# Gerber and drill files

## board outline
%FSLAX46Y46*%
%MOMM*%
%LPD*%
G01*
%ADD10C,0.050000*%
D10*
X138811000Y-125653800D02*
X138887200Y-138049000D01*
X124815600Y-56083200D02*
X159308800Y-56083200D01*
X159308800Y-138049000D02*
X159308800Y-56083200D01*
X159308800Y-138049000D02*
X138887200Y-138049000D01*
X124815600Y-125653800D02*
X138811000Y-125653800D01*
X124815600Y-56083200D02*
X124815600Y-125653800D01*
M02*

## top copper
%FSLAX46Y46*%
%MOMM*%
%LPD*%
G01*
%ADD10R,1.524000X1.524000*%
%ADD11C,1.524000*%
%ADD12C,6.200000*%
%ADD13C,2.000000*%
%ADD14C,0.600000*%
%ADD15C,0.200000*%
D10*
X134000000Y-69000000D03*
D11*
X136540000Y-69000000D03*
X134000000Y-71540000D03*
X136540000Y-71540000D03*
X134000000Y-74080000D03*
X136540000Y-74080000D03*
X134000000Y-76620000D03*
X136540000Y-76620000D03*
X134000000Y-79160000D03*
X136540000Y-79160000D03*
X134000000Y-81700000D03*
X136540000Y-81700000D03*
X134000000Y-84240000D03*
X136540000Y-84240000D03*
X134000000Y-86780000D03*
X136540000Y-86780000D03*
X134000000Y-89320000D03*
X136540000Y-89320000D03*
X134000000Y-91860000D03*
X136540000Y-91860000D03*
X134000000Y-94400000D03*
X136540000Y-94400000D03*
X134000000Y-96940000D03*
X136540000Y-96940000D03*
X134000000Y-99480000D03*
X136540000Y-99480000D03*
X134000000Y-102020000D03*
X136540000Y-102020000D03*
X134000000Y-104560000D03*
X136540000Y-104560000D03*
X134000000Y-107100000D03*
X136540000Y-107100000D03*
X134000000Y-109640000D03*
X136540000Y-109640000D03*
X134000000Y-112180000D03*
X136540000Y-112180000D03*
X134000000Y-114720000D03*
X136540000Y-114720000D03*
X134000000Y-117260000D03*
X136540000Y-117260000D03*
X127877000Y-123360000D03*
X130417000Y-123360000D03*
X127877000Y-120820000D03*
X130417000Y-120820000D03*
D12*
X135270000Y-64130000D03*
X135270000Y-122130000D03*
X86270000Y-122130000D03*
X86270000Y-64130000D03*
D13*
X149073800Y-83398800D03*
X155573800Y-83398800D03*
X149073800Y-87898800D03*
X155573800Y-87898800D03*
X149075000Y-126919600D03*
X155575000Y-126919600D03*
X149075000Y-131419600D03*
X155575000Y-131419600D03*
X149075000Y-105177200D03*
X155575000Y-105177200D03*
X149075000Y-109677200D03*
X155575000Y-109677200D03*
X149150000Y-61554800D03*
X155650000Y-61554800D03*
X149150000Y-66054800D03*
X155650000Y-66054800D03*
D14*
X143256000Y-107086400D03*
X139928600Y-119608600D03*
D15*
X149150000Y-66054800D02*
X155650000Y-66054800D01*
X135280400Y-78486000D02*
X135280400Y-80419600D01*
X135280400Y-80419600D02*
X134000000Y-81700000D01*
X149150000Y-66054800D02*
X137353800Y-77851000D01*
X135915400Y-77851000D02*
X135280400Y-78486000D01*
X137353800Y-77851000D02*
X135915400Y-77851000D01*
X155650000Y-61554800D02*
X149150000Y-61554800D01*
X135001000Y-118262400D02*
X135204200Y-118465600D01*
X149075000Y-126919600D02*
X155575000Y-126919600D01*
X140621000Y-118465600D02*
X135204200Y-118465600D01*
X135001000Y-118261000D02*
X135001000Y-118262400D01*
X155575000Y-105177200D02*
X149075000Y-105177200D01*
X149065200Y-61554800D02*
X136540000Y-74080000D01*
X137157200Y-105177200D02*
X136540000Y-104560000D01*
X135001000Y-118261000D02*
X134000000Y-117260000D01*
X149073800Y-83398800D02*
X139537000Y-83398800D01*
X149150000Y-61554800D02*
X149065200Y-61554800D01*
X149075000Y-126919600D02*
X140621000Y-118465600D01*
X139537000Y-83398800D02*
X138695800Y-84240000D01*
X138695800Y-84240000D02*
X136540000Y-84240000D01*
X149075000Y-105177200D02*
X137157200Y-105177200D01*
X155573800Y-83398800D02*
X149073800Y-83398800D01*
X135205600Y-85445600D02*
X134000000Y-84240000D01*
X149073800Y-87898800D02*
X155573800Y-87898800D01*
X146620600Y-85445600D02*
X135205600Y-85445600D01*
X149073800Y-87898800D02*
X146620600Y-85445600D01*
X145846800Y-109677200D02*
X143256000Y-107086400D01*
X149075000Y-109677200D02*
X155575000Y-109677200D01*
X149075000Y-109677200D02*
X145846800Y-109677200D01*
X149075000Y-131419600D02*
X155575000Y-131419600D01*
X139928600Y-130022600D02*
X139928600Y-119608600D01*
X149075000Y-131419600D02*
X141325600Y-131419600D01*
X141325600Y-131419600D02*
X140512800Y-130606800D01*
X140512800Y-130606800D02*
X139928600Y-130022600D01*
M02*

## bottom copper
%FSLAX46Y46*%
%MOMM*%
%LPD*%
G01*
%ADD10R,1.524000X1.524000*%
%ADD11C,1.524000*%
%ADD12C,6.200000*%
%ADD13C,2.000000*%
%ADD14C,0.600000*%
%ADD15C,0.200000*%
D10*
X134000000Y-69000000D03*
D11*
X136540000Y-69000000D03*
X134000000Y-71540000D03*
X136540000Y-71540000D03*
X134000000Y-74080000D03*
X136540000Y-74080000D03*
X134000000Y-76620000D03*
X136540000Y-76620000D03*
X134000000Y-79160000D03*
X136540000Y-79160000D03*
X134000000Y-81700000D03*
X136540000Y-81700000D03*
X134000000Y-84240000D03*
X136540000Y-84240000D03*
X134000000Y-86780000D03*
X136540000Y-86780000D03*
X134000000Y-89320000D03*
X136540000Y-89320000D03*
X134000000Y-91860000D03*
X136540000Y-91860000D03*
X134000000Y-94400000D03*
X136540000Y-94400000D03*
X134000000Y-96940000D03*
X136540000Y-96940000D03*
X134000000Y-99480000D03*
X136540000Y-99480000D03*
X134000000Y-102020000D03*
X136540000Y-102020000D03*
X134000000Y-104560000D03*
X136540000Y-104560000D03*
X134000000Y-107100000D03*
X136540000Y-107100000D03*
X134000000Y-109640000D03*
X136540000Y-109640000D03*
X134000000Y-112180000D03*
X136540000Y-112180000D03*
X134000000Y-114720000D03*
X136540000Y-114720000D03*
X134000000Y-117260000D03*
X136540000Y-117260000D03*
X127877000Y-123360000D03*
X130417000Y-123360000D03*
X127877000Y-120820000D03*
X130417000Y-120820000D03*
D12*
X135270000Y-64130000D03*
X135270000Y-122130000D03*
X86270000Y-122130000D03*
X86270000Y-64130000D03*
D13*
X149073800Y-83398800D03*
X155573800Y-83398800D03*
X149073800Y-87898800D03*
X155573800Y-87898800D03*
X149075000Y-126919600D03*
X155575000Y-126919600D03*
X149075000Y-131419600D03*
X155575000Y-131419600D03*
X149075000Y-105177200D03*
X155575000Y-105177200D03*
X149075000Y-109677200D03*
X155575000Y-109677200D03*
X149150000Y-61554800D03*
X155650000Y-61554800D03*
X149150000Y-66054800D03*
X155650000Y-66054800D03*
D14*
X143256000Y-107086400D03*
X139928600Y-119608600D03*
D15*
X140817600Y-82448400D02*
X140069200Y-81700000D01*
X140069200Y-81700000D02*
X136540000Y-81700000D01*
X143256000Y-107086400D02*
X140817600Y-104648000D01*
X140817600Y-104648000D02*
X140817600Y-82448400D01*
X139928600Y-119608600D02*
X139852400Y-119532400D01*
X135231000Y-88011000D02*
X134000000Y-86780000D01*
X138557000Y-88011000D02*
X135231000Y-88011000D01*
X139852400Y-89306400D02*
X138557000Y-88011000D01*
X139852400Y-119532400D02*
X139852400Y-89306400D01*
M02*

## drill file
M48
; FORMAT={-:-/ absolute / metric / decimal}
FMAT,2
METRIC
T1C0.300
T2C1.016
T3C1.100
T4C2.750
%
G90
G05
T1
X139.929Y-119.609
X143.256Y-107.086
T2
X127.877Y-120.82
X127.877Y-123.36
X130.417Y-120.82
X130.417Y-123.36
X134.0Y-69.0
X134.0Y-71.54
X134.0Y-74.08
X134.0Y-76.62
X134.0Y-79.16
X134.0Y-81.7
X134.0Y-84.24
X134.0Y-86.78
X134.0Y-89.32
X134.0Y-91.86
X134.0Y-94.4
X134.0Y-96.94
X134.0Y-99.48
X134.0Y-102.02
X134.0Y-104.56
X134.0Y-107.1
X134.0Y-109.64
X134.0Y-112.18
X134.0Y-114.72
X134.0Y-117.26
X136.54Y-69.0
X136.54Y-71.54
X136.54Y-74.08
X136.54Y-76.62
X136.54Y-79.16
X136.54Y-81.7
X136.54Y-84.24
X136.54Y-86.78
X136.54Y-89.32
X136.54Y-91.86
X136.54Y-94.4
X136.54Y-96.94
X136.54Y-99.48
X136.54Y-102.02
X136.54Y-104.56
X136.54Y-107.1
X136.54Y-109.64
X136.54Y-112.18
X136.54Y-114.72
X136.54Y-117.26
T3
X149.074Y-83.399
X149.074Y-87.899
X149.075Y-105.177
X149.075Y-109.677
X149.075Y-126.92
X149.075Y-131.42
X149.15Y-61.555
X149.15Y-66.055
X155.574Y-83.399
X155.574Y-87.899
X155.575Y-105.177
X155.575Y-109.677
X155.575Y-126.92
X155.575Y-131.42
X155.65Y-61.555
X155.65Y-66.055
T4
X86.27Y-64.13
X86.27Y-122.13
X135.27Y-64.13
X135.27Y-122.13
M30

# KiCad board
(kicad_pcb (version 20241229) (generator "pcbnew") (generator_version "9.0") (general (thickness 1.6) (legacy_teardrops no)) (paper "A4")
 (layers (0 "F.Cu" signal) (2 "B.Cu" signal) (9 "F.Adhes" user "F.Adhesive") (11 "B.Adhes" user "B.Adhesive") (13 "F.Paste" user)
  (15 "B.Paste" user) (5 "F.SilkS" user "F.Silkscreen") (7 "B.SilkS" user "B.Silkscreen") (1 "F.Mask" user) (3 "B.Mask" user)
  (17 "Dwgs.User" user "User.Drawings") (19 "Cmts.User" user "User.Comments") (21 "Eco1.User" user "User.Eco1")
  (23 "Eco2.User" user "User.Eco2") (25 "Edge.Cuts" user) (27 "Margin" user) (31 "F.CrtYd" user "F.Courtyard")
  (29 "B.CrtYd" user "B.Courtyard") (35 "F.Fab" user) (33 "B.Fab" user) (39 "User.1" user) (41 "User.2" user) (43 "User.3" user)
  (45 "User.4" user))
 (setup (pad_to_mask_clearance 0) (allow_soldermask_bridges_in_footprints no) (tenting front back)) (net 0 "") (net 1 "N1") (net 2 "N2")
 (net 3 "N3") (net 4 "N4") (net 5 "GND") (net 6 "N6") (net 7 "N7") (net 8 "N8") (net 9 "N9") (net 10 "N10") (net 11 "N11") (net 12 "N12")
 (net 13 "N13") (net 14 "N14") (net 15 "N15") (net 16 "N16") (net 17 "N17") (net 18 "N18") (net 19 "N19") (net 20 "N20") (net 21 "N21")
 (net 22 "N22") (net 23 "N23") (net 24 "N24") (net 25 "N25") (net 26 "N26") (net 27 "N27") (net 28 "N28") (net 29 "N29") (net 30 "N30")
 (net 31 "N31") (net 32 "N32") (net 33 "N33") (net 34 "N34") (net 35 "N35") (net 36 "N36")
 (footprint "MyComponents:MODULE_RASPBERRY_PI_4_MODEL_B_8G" (layer "F.Cu") (at 110.77 103.13 -90)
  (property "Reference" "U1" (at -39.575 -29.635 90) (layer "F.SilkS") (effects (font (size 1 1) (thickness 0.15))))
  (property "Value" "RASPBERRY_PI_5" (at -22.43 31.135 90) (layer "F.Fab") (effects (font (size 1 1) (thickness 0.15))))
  (pad "1" thru_hole rect (at -34.13 -23.23 270) (size 1.524 1.524) (drill 1.016) (layers "*.Cu" "*.Mask") (remove_unused_layers no)
   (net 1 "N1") (solder_mask_margin 0.102))
  (pad "2" thru_hole circle (at -34.13 -25.77 270) (size 1.524 1.524) (drill 1.016) (layers "*.Cu" "*.Mask") (remove_unused_layers no)
   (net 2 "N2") (solder_mask_margin 0.102))
  (pad "3" thru_hole circle (at -31.59 -23.23 270) (size 1.524 1.524) (drill 1.016) (layers "*.Cu" "*.Mask") (remove_unused_layers no)
   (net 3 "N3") (solder_mask_margin 0.102))
  (pad "4" thru_hole circle (at -31.59 -25.77 270) (size 1.524 1.524) (drill 1.016) (layers "*.Cu" "*.Mask") (remove_unused_layers no)
   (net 2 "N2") (solder_mask_margin 0.102))
  (pad "5" thru_hole circle (at -29.05 -23.23 270) (size 1.524 1.524) (drill 1.016) (layers "*.Cu" "*.Mask") (remove_unused_layers no)
   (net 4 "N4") (solder_mask_margin 0.102))
  (pad "6" thru_hole circle (at -29.05 -25.77 270) (size 1.524 1.524) (drill 1.016) (layers "*.Cu" "*.Mask") (remove_unused_layers no)
   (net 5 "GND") (solder_mask_margin 0.102))
  (pad "7" thru_hole circle (at -26.51 -23.23 270) (size 1.524 1.524) (drill 1.016) (layers "*.Cu" "*.Mask") (remove_unused_layers no)
   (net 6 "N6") (solder_mask_margin 0.102))
  (pad "8" thru_hole circle (at -26.51 -25.77 270) (size 1.524 1.524) (drill 1.016) (layers "*.Cu" "*.Mask") (remove_unused_layers no)
   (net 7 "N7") (solder_mask_margin 0.102))
  (pad "9" thru_hole circle (at -23.97 -23.23 270) (size 1.524 1.524) (drill 1.016) (layers "*.Cu" "*.Mask") (remove_unused_layers no)
   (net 5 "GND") (solder_mask_margin 0.102))
  (pad "10" thru_hole circle (at -23.97 -25.77 270) (size 1.524 1.524) (drill 1.016) (layers "*.Cu" "*.Mask") (remove_unused_layers no)
   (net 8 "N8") (solder_mask_margin 0.102))
  (pad "11" thru_hole circle (at -21.43 -23.23 270) (size 1.524 1.524) (drill 1.016) (layers "*.Cu" "*.Mask") (remove_unused_layers no)
   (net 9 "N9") (solder_mask_margin 0.102))
  (pad "12" thru_hole circle (at -21.43 -25.77 270) (size 1.524 1.524) (drill 1.016) (layers "*.Cu" "*.Mask") (remove_unused_layers no)
   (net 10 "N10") (solder_mask_margin 0.102))
  (pad "13" thru_hole circle (at -18.89 -23.23 270) (size 1.524 1.524) (drill 1.016) (layers "*.Cu" "*.Mask") (remove_unused_layers no)
   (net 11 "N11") (solder_mask_margin 0.102))
  (pad "14" thru_hole circle (at -18.89 -25.77 270) (size 1.524 1.524) (drill 1.016) (layers "*.Cu" "*.Mask") (remove_unused_layers no)
   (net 5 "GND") (solder_mask_margin 0.102))
  (pad "15" thru_hole circle (at -16.35 -23.23 270) (size 1.524 1.524) (drill 1.016) (layers "*.Cu" "*.Mask") (remove_unused_layers no)
   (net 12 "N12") (solder_mask_margin 0.102))
  (pad "16" thru_hole circle (at -16.35 -25.77 270) (size 1.524 1.524) (drill 1.016) (layers "*.Cu" "*.Mask") (remove_unused_layers no)
   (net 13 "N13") (solder_mask_margin 0.102))
  (pad "17" thru_hole circle (at -13.81 -23.23 270) (size 1.524 1.524) (drill 1.016) (layers "*.Cu" "*.Mask") (remove_unused_layers no)
   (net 1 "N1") (solder_mask_margin 0.102))
  (pad "18" thru_hole circle (at -13.81 -25.77 270) (size 1.524 1.524) (drill 1.016) (layers "*.Cu" "*.Mask") (remove_unused_layers no)
   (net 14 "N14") (solder_mask_margin 0.102))
  (pad "19" thru_hole circle (at -11.27 -23.23 270) (size 1.524 1.524) (drill 1.016) (layers "*.Cu" "*.Mask") (remove_unused_layers no)
   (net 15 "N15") (solder_mask_margin 0.102))
  (pad "20" thru_hole circle (at -11.27 -25.77 270) (size 1.524 1.524) (drill 1.016) (layers "*.Cu" "*.Mask") (remove_unused_layers no)
   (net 5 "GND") (solder_mask_margin 0.102))
  (pad "21" thru_hole circle (at -8.73 -23.23 270) (size 1.524 1.524) (drill 1.016) (layers "*.Cu" "*.Mask") (remove_unused_layers no)
   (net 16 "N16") (solder_mask_margin 0.102))
  (pad "22" thru_hole circle (at -8.73 -25.77 270) (size 1.524 1.524) (drill 1.016) (layers "*.Cu" "*.Mask") (remove_unused_layers no)
   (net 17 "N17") (solder_mask_margin 0.102))
  (pad "23" thru_hole circle (at -6.19 -23.23 270) (size 1.524 1.524) (drill 1.016) (layers "*.Cu" "*.Mask") (remove_unused_layers no)
   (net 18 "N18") (solder_mask_margin 0.102))
  (pad "24" thru_hole circle (at -6.19 -25.77 270) (size 1.524 1.524) (drill 1.016) (layers "*.Cu" "*.Mask") (remove_unused_layers no)
   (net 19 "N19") (solder_mask_margin 0.102))
  (pad "25" thru_hole circle (at -3.65 -23.23 270) (size 1.524 1.524) (drill 1.016) (layers "*.Cu" "*.Mask") (remove_unused_layers no)
   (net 5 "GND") (solder_mask_margin 0.102))
  (pad "26" thru_hole circle (at -3.65 -25.77 270) (size 1.524 1.524) (drill 1.016) (layers "*.Cu" "*.Mask") (remove_unused_layers no)
   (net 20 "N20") (solder_mask_margin 0.102))
  (pad "27" thru_hole circle (at -1.11 -23.23 270) (size 1.524 1.524) (drill 1.016) (layers "*.Cu" "*.Mask") (remove_unused_layers no)
   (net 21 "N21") (solder_mask_margin 0.102))
  (pad "28" thru_hole circle (at -1.11 -25.77 270) (size 1.524 1.524) (drill 1.016) (layers "*.Cu" "*.Mask") (remove_unused_layers no)
   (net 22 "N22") (solder_mask_margin 0.102))
  (pad "29" thru_hole circle (at 1.43 -23.23 270) (size 1.524 1.524) (drill 1.016) (layers "*.Cu" "*.Mask") (remove_unused_layers no)
   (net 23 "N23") (solder_mask_margin 0.102))
  (pad "30" thru_hole circle (at 1.43 -25.77 270) (size 1.524 1.524) (drill 1.016) (layers "*.Cu" "*.Mask") (remove_unused_layers no)
   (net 5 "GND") (solder_mask_margin 0.102))
  (pad "31" thru_hole circle (at 3.97 -23.23 270) (size 1.524 1.524) (drill 1.016) (layers "*.Cu" "*.Mask") (remove_unused_layers no)
   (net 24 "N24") (solder_mask_margin 0.102))
  (pad "32" thru_hole circle (at 3.97 -25.77 270) (size 1.524 1.524) (drill 1.016) (layers "*.Cu" "*.Mask") (remove_unused_layers no)
   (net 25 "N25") (solder_mask_margin 0.102))
  (pad "33" thru_hole circle (at 6.51 -23.23 270) (size 1.524 1.524) (drill 1.016) (layers "*.Cu" "*.Mask") (remove_unused_layers no)
   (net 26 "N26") (solder_mask_margin 0.102))
  (pad "34" thru_hole circle (at 6.51 -25.77 270) (size 1.524 1.524) (drill 1.016) (layers "*.Cu" "*.Mask") (remove_unused_layers no)
   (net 5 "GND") (solder_mask_margin 0.102))
  (pad "35" thru_hole circle (at 9.05 -23.23 270) (size 1.524 1.524) (drill 1.016) (layers "*.Cu" "*.Mask") (remove_unused_layers no)
   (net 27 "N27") (solder_mask_margin 0.102))
  (pad "36" thru_hole circle (at 9.05 -25.77 270) (size 1.524 1.524) (drill 1.016) (layers "*.Cu" "*.Mask") (remove_unused_layers no)
   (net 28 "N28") (solder_mask_margin 0.102))
  (pad "37" thru_hole circle (at 11.59 -23.23 270) (size 1.524 1.524) (drill 1.016) (layers "*.Cu" "*.Mask") (remove_unused_layers no)
   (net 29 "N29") (solder_mask_margin 0.102))
  (pad "38" thru_hole circle (at 11.59 -25.77 270) (size 1.524 1.524) (drill 1.016) (layers "*.Cu" "*.Mask") (remove_unused_layers no)
   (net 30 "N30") (solder_mask_margin 0.102))
  (pad "39" thru_hole circle (at 14.13 -23.23 270) (size 1.524 1.524) (drill 1.016) (layers "*.Cu" "*.Mask") (remove_unused_layers no)
   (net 5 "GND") (solder_mask_margin 0.102))
  (pad "40" thru_hole circle (at 14.13 -25.77 270) (size 1.524 1.524) (drill 1.016) (layers "*.Cu" "*.Mask") (remove_unused_layers no)
   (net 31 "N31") (solder_mask_margin 0.102))
  (pad "41" thru_hole circle (at 20.23 -17.107 270) (size 1.524 1.524) (drill 1.016) (layers "*.Cu" "*.Mask") (remove_unused_layers no)
   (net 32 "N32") (solder_mask_margin 0.102))
  (pad "42" thru_hole circle (at 20.23 -19.647 270) (size 1.524 1.524) (drill 1.016) (layers "*.Cu" "*.Mask") (remove_unused_layers no)
   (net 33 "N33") (solder_mask_margin 0.102))
  (pad "43" thru_hole circle (at 17.69 -17.107 270) (size 1.524 1.524) (drill 1.016) (layers "*.Cu" "*.Mask") (remove_unused_layers no)
   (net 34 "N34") (solder_mask_margin 0.102))
  (pad "44" thru_hole circle (at 17.69 -19.647 270) (size 1.524 1.524) (drill 1.016) (layers "*.Cu" "*.Mask") (remove_unused_layers no)
   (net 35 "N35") (solder_mask_margin 0.102))
  (pad "S1" thru_hole circle (at -39 -24.5 270) (size 6.2 6.2) (drill 2.75) (layers "*.Cu" "*.Mask") (remove_unused_layers no)
   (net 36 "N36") (solder_mask_margin 0.102))
  (pad "S2" thru_hole circle (at 19 -24.5 270) (size 6.2 6.2) (drill 2.75) (layers "*.Cu" "*.Mask") (remove_unused_layers no) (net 36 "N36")
   (solder_mask_margin 0.102))
  (pad "S3" thru_hole circle (at 19 24.5 270) (size 6.2 6.2) (drill 2.75) (layers "*.Cu" "*.Mask") (remove_unused_layers no) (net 36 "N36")
   (solder_mask_margin 0.102))
  (pad "S4" thru_hole circle (at -39 24.5 270) (size 6.2 6.2) (drill 2.75) (layers "*.Cu" "*.Mask") (remove_unused_layers no) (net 36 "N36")
   (solder_mask_margin 0.102)))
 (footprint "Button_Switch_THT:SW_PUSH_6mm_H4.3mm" (layer "F.Cu") (at 149.0738 83.3988)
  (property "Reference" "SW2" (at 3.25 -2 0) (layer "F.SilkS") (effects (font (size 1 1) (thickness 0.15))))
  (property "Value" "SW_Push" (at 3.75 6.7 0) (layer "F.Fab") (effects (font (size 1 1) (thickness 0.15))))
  (pad "1" thru_hole circle (at 0 0 90) (size 2 2) (drill 1.1) (layers "*.Cu" "*.Mask") (remove_unused_layers no) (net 5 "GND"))
  (pad "1" thru_hole circle (at 6.5 0 90) (size 2 2) (drill 1.1) (layers "*.Cu" "*.Mask") (remove_unused_layers no) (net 5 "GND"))
  (pad "2" thru_hole circle (at 0 4.5 90) (size 2 2) (drill 1.1) (layers "*.Cu" "*.Mask") (remove_unused_layers no) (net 11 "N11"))
  (pad "2" thru_hole circle (at 6.5 4.5 90) (size 2 2) (drill 1.1) (layers "*.Cu" "*.Mask") (remove_unused_layers no) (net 11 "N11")))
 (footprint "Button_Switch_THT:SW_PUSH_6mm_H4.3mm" (layer "F.Cu") (at 149.075 126.9196)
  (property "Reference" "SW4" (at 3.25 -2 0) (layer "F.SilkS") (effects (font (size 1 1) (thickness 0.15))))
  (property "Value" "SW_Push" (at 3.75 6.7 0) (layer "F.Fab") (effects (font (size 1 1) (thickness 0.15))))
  (pad "1" thru_hole circle (at 0 0 90) (size 2 2) (drill 1.1) (layers "*.Cu" "*.Mask") (remove_unused_layers no) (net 5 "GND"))
  (pad "1" thru_hole circle (at 6.5 0 90) (size 2 2) (drill 1.1) (layers "*.Cu" "*.Mask") (remove_unused_layers no) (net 5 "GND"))
  (pad "2" thru_hole circle (at 0 4.5 90) (size 2 2) (drill 1.1) (layers "*.Cu" "*.Mask") (remove_unused_layers no) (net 12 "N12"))
  (pad "2" thru_hole circle (at 6.5 4.5 90) (size 2 2) (drill 1.1) (layers "*.Cu" "*.Mask") (remove_unused_layers no) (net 12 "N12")))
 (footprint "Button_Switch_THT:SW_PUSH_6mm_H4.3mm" (layer "F.Cu") (at 149.075 105.1772)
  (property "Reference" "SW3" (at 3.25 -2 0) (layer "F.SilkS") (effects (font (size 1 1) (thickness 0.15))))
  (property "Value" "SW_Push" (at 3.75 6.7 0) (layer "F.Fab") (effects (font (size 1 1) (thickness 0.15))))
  (pad "1" thru_hole circle (at 0 0 90) (size 2 2) (drill 1.1) (layers "*.Cu" "*.Mask") (remove_unused_layers no) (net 5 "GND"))
  (pad "1" thru_hole circle (at 6.5 0 90) (size 2 2) (drill 1.1) (layers "*.Cu" "*.Mask") (remove_unused_layers no) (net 5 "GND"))
  (pad "2" thru_hole circle (at 0 4.5 90) (size 2 2) (drill 1.1) (layers "*.Cu" "*.Mask") (remove_unused_layers no) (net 10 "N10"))
  (pad "2" thru_hole circle (at 6.5 4.5 90) (size 2 2) (drill 1.1) (layers "*.Cu" "*.Mask") (remove_unused_layers no) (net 10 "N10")))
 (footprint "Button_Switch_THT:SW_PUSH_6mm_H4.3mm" (layer "F.Cu") (at 149.15 61.5548)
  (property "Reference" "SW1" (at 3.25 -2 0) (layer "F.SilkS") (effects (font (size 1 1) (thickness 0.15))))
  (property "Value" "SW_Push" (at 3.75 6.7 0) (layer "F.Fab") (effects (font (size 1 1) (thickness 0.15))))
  (pad "1" thru_hole circle (at 0 0 90) (size 2 2) (drill 1.1) (layers "*.Cu" "*.Mask") (remove_unused_layers no) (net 5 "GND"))
  (pad "1" thru_hole circle (at 6.5 0 90) (size 2 2) (drill 1.1) (layers "*.Cu" "*.Mask") (remove_unused_layers no) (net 5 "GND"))
  (pad "2" thru_hole circle (at 0 4.5 90) (size 2 2) (drill 1.1) (layers "*.Cu" "*.Mask") (remove_unused_layers no) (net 9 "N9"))
  (pad "2" thru_hole circle (at 6.5 4.5 90) (size 2 2) (drill 1.1) (layers "*.Cu" "*.Mask") (remove_unused_layers no) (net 9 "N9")))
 (gr_line (start 138.811 125.6538) (end 138.8872 138.049) (stroke (width 0.05) (type default)) (layer "Edge.Cuts"))
 (gr_line (start 124.8156 56.0832) (end 159.3088 56.0832) (stroke (width 0.05) (type default)) (layer "Edge.Cuts"))
 (gr_line (start 159.3088 138.049) (end 159.3088 56.0832) (stroke (width 0.05) (type default)) (layer "Edge.Cuts"))
 (gr_line (start 159.3088 138.049) (end 138.8872 138.049) (stroke (width 0.05) (type default)) (layer "Edge.Cuts"))
 (gr_line (start 124.8156 125.6538) (end 138.811 125.6538) (stroke (width 0.05) (type default)) (layer "Edge.Cuts"))
 (gr_line (start 124.8156 56.0832) (end 124.8156 125.6538) (stroke (width 0.05) (type default)) (layer "Edge.Cuts"))
 (segment (start 149.15 66.0548) (end 155.65 66.0548) (width 0.2) (layer "F.Cu") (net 9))
 (segment (start 135.2804 78.486) (end 135.2804 80.4196) (width 0.2) (layer "F.Cu") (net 9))
 (segment (start 135.2804 80.4196) (end 134 81.7) (width 0.2) (layer "F.Cu") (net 9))
 (segment (start 149.15 66.0548) (end 137.3538 77.851) (width 0.2) (layer "F.Cu") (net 9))
 (segment (start 135.9154 77.851) (end 135.2804 78.486) (width 0.2) (layer "F.Cu") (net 9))
 (segment (start 137.3538 77.851) (end 135.9154 77.851) (width 0.2) (layer "F.Cu") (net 9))
 (segment (start 155.65 61.5548) (end 149.15 61.5548) (width 0.2) (layer "F.Cu") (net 5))
 (segment (start 135.001 118.2624) (end 135.2042 118.4656) (width 0.2) (layer "F.Cu") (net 5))
 (segment (start 149.075 126.9196) (end 155.575 126.9196) (width 0.2) (layer "F.Cu") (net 5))
 (segment (start 140.621 118.4656) (end 135.2042 118.4656) (width 0.2) (layer "F.Cu") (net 5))
 (segment (start 135.001 118.261) (end 135.001 118.2624) (width 0.2) (layer "F.Cu") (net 5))
 (segment (start 155.575 105.1772) (end 149.075 105.1772) (width 0.2) (layer "F.Cu") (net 5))
 (segment (start 149.0652 61.5548) (end 136.54 74.08) (width 0.2) (layer "F.Cu") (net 5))
 (segment (start 137.1572 105.1772) (end 136.54 104.56) (width 0.2) (layer "F.Cu") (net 5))
 (segment (start 135.001 118.261) (end 134 117.26) (width 0.2) (layer "F.Cu") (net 5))
 (segment (start 149.0738 83.3988) (end 139.537 83.3988) (width 0.2) (layer "F.Cu") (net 5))
 (segment (start 149.15 61.5548) (end 149.0652 61.5548) (width 0.2) (layer "F.Cu") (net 5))
 (segment (start 149.075 126.9196) (end 140.621 118.4656) (width 0.2) (layer "F.Cu") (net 5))
 (segment (start 139.537 83.3988) (end 138.6958 84.24) (width 0.2) (layer "F.Cu") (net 5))
 (segment (start 138.6958 84.24) (end 136.54 84.24) (width 0.2) (layer "F.Cu") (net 5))
 (segment (start 149.075 105.1772) (end 137.1572 105.1772) (width 0.2) (layer "F.Cu") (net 5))
 (segment (start 155.5738 83.3988) (end 149.0738 83.3988) (width 0.2) (layer "F.Cu") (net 5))
 (segment (start 135.2056 85.4456) (end 134 84.24) (width 0.2) (layer "F.Cu") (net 11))
 (segment (start 149.0738 87.8988) (end 155.5738 87.8988) (width 0.2) (layer "F.Cu") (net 11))
 (segment (start 146.6206 85.4456) (end 135.2056 85.4456) (width 0.2) (layer "F.Cu") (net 11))
 (segment (start 149.0738 87.8988) (end 146.6206 85.4456) (width 0.2) (layer "F.Cu") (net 11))
 (segment (start 145.8468 109.6772) (end 143.256 107.0864) (width 0.2) (layer "F.Cu") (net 10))
 (segment (start 149.075 109.6772) (end 155.575 109.6772) (width 0.2) (layer "F.Cu") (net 10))
 (segment (start 149.075 109.6772) (end 145.8468 109.6772) (width 0.2) (layer "F.Cu") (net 10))
 (via (at 143.256 107.0864) (size 0.6) (drill 0.3) (layers "F.Cu" "B.Cu") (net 10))
 (segment (start 140.8176 82.4484) (end 140.0692 81.7) (width 0.2) (layer "B.Cu") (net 10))
 (segment (start 140.0692 81.7) (end 136.54 81.7) (width 0.2) (layer "B.Cu") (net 10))
 (segment (start 143.256 107.0864) (end 140.8176 104.648) (width 0.2) (layer "B.Cu") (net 10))
 (segment (start 140.8176 104.648) (end 140.8176 82.4484) (width 0.2) (layer "B.Cu") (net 10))
 (segment (start 149.075 131.4196) (end 155.575 131.4196) (width 0.2) (layer "F.Cu") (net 12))
 (segment (start 139.9286 130.0226) (end 139.9286 119.6086) (width 0.2) (layer "F.Cu") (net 12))
 (segment (start 149.075 131.4196) (end 141.3256 131.4196) (width 0.2) (layer "F.Cu") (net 12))
 (segment (start 141.3256 131.4196) (end 140.5128 130.6068) (width 0.2) (layer "F.Cu") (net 12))
 (segment (start 140.5128 130.6068) (end 139.9286 130.0226) (width 0.2) (layer "F.Cu") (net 12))
 (via (at 139.9286 119.6086) (size 0.6) (drill 0.3) (layers "F.Cu" "B.Cu") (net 12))
 (segment (start 139.9286 119.6086) (end 139.8524 119.5324) (width 0.2) (layer "B.Cu") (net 12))
 (segment (start 135.231 88.011) (end 134 86.78) (width 0.2) (layer "B.Cu") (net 12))
 (segment (start 138.557 88.011) (end 135.231 88.011) (width 0.2) (layer "B.Cu") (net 12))
 (segment (start 139.8524 89.3064) (end 138.557 88.011) (width 0.2) (layer "B.Cu") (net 12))
 (segment (start 139.8524 119.5324) (end 139.8524 89.3064) (width 0.2) (layer "B.Cu") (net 12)))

